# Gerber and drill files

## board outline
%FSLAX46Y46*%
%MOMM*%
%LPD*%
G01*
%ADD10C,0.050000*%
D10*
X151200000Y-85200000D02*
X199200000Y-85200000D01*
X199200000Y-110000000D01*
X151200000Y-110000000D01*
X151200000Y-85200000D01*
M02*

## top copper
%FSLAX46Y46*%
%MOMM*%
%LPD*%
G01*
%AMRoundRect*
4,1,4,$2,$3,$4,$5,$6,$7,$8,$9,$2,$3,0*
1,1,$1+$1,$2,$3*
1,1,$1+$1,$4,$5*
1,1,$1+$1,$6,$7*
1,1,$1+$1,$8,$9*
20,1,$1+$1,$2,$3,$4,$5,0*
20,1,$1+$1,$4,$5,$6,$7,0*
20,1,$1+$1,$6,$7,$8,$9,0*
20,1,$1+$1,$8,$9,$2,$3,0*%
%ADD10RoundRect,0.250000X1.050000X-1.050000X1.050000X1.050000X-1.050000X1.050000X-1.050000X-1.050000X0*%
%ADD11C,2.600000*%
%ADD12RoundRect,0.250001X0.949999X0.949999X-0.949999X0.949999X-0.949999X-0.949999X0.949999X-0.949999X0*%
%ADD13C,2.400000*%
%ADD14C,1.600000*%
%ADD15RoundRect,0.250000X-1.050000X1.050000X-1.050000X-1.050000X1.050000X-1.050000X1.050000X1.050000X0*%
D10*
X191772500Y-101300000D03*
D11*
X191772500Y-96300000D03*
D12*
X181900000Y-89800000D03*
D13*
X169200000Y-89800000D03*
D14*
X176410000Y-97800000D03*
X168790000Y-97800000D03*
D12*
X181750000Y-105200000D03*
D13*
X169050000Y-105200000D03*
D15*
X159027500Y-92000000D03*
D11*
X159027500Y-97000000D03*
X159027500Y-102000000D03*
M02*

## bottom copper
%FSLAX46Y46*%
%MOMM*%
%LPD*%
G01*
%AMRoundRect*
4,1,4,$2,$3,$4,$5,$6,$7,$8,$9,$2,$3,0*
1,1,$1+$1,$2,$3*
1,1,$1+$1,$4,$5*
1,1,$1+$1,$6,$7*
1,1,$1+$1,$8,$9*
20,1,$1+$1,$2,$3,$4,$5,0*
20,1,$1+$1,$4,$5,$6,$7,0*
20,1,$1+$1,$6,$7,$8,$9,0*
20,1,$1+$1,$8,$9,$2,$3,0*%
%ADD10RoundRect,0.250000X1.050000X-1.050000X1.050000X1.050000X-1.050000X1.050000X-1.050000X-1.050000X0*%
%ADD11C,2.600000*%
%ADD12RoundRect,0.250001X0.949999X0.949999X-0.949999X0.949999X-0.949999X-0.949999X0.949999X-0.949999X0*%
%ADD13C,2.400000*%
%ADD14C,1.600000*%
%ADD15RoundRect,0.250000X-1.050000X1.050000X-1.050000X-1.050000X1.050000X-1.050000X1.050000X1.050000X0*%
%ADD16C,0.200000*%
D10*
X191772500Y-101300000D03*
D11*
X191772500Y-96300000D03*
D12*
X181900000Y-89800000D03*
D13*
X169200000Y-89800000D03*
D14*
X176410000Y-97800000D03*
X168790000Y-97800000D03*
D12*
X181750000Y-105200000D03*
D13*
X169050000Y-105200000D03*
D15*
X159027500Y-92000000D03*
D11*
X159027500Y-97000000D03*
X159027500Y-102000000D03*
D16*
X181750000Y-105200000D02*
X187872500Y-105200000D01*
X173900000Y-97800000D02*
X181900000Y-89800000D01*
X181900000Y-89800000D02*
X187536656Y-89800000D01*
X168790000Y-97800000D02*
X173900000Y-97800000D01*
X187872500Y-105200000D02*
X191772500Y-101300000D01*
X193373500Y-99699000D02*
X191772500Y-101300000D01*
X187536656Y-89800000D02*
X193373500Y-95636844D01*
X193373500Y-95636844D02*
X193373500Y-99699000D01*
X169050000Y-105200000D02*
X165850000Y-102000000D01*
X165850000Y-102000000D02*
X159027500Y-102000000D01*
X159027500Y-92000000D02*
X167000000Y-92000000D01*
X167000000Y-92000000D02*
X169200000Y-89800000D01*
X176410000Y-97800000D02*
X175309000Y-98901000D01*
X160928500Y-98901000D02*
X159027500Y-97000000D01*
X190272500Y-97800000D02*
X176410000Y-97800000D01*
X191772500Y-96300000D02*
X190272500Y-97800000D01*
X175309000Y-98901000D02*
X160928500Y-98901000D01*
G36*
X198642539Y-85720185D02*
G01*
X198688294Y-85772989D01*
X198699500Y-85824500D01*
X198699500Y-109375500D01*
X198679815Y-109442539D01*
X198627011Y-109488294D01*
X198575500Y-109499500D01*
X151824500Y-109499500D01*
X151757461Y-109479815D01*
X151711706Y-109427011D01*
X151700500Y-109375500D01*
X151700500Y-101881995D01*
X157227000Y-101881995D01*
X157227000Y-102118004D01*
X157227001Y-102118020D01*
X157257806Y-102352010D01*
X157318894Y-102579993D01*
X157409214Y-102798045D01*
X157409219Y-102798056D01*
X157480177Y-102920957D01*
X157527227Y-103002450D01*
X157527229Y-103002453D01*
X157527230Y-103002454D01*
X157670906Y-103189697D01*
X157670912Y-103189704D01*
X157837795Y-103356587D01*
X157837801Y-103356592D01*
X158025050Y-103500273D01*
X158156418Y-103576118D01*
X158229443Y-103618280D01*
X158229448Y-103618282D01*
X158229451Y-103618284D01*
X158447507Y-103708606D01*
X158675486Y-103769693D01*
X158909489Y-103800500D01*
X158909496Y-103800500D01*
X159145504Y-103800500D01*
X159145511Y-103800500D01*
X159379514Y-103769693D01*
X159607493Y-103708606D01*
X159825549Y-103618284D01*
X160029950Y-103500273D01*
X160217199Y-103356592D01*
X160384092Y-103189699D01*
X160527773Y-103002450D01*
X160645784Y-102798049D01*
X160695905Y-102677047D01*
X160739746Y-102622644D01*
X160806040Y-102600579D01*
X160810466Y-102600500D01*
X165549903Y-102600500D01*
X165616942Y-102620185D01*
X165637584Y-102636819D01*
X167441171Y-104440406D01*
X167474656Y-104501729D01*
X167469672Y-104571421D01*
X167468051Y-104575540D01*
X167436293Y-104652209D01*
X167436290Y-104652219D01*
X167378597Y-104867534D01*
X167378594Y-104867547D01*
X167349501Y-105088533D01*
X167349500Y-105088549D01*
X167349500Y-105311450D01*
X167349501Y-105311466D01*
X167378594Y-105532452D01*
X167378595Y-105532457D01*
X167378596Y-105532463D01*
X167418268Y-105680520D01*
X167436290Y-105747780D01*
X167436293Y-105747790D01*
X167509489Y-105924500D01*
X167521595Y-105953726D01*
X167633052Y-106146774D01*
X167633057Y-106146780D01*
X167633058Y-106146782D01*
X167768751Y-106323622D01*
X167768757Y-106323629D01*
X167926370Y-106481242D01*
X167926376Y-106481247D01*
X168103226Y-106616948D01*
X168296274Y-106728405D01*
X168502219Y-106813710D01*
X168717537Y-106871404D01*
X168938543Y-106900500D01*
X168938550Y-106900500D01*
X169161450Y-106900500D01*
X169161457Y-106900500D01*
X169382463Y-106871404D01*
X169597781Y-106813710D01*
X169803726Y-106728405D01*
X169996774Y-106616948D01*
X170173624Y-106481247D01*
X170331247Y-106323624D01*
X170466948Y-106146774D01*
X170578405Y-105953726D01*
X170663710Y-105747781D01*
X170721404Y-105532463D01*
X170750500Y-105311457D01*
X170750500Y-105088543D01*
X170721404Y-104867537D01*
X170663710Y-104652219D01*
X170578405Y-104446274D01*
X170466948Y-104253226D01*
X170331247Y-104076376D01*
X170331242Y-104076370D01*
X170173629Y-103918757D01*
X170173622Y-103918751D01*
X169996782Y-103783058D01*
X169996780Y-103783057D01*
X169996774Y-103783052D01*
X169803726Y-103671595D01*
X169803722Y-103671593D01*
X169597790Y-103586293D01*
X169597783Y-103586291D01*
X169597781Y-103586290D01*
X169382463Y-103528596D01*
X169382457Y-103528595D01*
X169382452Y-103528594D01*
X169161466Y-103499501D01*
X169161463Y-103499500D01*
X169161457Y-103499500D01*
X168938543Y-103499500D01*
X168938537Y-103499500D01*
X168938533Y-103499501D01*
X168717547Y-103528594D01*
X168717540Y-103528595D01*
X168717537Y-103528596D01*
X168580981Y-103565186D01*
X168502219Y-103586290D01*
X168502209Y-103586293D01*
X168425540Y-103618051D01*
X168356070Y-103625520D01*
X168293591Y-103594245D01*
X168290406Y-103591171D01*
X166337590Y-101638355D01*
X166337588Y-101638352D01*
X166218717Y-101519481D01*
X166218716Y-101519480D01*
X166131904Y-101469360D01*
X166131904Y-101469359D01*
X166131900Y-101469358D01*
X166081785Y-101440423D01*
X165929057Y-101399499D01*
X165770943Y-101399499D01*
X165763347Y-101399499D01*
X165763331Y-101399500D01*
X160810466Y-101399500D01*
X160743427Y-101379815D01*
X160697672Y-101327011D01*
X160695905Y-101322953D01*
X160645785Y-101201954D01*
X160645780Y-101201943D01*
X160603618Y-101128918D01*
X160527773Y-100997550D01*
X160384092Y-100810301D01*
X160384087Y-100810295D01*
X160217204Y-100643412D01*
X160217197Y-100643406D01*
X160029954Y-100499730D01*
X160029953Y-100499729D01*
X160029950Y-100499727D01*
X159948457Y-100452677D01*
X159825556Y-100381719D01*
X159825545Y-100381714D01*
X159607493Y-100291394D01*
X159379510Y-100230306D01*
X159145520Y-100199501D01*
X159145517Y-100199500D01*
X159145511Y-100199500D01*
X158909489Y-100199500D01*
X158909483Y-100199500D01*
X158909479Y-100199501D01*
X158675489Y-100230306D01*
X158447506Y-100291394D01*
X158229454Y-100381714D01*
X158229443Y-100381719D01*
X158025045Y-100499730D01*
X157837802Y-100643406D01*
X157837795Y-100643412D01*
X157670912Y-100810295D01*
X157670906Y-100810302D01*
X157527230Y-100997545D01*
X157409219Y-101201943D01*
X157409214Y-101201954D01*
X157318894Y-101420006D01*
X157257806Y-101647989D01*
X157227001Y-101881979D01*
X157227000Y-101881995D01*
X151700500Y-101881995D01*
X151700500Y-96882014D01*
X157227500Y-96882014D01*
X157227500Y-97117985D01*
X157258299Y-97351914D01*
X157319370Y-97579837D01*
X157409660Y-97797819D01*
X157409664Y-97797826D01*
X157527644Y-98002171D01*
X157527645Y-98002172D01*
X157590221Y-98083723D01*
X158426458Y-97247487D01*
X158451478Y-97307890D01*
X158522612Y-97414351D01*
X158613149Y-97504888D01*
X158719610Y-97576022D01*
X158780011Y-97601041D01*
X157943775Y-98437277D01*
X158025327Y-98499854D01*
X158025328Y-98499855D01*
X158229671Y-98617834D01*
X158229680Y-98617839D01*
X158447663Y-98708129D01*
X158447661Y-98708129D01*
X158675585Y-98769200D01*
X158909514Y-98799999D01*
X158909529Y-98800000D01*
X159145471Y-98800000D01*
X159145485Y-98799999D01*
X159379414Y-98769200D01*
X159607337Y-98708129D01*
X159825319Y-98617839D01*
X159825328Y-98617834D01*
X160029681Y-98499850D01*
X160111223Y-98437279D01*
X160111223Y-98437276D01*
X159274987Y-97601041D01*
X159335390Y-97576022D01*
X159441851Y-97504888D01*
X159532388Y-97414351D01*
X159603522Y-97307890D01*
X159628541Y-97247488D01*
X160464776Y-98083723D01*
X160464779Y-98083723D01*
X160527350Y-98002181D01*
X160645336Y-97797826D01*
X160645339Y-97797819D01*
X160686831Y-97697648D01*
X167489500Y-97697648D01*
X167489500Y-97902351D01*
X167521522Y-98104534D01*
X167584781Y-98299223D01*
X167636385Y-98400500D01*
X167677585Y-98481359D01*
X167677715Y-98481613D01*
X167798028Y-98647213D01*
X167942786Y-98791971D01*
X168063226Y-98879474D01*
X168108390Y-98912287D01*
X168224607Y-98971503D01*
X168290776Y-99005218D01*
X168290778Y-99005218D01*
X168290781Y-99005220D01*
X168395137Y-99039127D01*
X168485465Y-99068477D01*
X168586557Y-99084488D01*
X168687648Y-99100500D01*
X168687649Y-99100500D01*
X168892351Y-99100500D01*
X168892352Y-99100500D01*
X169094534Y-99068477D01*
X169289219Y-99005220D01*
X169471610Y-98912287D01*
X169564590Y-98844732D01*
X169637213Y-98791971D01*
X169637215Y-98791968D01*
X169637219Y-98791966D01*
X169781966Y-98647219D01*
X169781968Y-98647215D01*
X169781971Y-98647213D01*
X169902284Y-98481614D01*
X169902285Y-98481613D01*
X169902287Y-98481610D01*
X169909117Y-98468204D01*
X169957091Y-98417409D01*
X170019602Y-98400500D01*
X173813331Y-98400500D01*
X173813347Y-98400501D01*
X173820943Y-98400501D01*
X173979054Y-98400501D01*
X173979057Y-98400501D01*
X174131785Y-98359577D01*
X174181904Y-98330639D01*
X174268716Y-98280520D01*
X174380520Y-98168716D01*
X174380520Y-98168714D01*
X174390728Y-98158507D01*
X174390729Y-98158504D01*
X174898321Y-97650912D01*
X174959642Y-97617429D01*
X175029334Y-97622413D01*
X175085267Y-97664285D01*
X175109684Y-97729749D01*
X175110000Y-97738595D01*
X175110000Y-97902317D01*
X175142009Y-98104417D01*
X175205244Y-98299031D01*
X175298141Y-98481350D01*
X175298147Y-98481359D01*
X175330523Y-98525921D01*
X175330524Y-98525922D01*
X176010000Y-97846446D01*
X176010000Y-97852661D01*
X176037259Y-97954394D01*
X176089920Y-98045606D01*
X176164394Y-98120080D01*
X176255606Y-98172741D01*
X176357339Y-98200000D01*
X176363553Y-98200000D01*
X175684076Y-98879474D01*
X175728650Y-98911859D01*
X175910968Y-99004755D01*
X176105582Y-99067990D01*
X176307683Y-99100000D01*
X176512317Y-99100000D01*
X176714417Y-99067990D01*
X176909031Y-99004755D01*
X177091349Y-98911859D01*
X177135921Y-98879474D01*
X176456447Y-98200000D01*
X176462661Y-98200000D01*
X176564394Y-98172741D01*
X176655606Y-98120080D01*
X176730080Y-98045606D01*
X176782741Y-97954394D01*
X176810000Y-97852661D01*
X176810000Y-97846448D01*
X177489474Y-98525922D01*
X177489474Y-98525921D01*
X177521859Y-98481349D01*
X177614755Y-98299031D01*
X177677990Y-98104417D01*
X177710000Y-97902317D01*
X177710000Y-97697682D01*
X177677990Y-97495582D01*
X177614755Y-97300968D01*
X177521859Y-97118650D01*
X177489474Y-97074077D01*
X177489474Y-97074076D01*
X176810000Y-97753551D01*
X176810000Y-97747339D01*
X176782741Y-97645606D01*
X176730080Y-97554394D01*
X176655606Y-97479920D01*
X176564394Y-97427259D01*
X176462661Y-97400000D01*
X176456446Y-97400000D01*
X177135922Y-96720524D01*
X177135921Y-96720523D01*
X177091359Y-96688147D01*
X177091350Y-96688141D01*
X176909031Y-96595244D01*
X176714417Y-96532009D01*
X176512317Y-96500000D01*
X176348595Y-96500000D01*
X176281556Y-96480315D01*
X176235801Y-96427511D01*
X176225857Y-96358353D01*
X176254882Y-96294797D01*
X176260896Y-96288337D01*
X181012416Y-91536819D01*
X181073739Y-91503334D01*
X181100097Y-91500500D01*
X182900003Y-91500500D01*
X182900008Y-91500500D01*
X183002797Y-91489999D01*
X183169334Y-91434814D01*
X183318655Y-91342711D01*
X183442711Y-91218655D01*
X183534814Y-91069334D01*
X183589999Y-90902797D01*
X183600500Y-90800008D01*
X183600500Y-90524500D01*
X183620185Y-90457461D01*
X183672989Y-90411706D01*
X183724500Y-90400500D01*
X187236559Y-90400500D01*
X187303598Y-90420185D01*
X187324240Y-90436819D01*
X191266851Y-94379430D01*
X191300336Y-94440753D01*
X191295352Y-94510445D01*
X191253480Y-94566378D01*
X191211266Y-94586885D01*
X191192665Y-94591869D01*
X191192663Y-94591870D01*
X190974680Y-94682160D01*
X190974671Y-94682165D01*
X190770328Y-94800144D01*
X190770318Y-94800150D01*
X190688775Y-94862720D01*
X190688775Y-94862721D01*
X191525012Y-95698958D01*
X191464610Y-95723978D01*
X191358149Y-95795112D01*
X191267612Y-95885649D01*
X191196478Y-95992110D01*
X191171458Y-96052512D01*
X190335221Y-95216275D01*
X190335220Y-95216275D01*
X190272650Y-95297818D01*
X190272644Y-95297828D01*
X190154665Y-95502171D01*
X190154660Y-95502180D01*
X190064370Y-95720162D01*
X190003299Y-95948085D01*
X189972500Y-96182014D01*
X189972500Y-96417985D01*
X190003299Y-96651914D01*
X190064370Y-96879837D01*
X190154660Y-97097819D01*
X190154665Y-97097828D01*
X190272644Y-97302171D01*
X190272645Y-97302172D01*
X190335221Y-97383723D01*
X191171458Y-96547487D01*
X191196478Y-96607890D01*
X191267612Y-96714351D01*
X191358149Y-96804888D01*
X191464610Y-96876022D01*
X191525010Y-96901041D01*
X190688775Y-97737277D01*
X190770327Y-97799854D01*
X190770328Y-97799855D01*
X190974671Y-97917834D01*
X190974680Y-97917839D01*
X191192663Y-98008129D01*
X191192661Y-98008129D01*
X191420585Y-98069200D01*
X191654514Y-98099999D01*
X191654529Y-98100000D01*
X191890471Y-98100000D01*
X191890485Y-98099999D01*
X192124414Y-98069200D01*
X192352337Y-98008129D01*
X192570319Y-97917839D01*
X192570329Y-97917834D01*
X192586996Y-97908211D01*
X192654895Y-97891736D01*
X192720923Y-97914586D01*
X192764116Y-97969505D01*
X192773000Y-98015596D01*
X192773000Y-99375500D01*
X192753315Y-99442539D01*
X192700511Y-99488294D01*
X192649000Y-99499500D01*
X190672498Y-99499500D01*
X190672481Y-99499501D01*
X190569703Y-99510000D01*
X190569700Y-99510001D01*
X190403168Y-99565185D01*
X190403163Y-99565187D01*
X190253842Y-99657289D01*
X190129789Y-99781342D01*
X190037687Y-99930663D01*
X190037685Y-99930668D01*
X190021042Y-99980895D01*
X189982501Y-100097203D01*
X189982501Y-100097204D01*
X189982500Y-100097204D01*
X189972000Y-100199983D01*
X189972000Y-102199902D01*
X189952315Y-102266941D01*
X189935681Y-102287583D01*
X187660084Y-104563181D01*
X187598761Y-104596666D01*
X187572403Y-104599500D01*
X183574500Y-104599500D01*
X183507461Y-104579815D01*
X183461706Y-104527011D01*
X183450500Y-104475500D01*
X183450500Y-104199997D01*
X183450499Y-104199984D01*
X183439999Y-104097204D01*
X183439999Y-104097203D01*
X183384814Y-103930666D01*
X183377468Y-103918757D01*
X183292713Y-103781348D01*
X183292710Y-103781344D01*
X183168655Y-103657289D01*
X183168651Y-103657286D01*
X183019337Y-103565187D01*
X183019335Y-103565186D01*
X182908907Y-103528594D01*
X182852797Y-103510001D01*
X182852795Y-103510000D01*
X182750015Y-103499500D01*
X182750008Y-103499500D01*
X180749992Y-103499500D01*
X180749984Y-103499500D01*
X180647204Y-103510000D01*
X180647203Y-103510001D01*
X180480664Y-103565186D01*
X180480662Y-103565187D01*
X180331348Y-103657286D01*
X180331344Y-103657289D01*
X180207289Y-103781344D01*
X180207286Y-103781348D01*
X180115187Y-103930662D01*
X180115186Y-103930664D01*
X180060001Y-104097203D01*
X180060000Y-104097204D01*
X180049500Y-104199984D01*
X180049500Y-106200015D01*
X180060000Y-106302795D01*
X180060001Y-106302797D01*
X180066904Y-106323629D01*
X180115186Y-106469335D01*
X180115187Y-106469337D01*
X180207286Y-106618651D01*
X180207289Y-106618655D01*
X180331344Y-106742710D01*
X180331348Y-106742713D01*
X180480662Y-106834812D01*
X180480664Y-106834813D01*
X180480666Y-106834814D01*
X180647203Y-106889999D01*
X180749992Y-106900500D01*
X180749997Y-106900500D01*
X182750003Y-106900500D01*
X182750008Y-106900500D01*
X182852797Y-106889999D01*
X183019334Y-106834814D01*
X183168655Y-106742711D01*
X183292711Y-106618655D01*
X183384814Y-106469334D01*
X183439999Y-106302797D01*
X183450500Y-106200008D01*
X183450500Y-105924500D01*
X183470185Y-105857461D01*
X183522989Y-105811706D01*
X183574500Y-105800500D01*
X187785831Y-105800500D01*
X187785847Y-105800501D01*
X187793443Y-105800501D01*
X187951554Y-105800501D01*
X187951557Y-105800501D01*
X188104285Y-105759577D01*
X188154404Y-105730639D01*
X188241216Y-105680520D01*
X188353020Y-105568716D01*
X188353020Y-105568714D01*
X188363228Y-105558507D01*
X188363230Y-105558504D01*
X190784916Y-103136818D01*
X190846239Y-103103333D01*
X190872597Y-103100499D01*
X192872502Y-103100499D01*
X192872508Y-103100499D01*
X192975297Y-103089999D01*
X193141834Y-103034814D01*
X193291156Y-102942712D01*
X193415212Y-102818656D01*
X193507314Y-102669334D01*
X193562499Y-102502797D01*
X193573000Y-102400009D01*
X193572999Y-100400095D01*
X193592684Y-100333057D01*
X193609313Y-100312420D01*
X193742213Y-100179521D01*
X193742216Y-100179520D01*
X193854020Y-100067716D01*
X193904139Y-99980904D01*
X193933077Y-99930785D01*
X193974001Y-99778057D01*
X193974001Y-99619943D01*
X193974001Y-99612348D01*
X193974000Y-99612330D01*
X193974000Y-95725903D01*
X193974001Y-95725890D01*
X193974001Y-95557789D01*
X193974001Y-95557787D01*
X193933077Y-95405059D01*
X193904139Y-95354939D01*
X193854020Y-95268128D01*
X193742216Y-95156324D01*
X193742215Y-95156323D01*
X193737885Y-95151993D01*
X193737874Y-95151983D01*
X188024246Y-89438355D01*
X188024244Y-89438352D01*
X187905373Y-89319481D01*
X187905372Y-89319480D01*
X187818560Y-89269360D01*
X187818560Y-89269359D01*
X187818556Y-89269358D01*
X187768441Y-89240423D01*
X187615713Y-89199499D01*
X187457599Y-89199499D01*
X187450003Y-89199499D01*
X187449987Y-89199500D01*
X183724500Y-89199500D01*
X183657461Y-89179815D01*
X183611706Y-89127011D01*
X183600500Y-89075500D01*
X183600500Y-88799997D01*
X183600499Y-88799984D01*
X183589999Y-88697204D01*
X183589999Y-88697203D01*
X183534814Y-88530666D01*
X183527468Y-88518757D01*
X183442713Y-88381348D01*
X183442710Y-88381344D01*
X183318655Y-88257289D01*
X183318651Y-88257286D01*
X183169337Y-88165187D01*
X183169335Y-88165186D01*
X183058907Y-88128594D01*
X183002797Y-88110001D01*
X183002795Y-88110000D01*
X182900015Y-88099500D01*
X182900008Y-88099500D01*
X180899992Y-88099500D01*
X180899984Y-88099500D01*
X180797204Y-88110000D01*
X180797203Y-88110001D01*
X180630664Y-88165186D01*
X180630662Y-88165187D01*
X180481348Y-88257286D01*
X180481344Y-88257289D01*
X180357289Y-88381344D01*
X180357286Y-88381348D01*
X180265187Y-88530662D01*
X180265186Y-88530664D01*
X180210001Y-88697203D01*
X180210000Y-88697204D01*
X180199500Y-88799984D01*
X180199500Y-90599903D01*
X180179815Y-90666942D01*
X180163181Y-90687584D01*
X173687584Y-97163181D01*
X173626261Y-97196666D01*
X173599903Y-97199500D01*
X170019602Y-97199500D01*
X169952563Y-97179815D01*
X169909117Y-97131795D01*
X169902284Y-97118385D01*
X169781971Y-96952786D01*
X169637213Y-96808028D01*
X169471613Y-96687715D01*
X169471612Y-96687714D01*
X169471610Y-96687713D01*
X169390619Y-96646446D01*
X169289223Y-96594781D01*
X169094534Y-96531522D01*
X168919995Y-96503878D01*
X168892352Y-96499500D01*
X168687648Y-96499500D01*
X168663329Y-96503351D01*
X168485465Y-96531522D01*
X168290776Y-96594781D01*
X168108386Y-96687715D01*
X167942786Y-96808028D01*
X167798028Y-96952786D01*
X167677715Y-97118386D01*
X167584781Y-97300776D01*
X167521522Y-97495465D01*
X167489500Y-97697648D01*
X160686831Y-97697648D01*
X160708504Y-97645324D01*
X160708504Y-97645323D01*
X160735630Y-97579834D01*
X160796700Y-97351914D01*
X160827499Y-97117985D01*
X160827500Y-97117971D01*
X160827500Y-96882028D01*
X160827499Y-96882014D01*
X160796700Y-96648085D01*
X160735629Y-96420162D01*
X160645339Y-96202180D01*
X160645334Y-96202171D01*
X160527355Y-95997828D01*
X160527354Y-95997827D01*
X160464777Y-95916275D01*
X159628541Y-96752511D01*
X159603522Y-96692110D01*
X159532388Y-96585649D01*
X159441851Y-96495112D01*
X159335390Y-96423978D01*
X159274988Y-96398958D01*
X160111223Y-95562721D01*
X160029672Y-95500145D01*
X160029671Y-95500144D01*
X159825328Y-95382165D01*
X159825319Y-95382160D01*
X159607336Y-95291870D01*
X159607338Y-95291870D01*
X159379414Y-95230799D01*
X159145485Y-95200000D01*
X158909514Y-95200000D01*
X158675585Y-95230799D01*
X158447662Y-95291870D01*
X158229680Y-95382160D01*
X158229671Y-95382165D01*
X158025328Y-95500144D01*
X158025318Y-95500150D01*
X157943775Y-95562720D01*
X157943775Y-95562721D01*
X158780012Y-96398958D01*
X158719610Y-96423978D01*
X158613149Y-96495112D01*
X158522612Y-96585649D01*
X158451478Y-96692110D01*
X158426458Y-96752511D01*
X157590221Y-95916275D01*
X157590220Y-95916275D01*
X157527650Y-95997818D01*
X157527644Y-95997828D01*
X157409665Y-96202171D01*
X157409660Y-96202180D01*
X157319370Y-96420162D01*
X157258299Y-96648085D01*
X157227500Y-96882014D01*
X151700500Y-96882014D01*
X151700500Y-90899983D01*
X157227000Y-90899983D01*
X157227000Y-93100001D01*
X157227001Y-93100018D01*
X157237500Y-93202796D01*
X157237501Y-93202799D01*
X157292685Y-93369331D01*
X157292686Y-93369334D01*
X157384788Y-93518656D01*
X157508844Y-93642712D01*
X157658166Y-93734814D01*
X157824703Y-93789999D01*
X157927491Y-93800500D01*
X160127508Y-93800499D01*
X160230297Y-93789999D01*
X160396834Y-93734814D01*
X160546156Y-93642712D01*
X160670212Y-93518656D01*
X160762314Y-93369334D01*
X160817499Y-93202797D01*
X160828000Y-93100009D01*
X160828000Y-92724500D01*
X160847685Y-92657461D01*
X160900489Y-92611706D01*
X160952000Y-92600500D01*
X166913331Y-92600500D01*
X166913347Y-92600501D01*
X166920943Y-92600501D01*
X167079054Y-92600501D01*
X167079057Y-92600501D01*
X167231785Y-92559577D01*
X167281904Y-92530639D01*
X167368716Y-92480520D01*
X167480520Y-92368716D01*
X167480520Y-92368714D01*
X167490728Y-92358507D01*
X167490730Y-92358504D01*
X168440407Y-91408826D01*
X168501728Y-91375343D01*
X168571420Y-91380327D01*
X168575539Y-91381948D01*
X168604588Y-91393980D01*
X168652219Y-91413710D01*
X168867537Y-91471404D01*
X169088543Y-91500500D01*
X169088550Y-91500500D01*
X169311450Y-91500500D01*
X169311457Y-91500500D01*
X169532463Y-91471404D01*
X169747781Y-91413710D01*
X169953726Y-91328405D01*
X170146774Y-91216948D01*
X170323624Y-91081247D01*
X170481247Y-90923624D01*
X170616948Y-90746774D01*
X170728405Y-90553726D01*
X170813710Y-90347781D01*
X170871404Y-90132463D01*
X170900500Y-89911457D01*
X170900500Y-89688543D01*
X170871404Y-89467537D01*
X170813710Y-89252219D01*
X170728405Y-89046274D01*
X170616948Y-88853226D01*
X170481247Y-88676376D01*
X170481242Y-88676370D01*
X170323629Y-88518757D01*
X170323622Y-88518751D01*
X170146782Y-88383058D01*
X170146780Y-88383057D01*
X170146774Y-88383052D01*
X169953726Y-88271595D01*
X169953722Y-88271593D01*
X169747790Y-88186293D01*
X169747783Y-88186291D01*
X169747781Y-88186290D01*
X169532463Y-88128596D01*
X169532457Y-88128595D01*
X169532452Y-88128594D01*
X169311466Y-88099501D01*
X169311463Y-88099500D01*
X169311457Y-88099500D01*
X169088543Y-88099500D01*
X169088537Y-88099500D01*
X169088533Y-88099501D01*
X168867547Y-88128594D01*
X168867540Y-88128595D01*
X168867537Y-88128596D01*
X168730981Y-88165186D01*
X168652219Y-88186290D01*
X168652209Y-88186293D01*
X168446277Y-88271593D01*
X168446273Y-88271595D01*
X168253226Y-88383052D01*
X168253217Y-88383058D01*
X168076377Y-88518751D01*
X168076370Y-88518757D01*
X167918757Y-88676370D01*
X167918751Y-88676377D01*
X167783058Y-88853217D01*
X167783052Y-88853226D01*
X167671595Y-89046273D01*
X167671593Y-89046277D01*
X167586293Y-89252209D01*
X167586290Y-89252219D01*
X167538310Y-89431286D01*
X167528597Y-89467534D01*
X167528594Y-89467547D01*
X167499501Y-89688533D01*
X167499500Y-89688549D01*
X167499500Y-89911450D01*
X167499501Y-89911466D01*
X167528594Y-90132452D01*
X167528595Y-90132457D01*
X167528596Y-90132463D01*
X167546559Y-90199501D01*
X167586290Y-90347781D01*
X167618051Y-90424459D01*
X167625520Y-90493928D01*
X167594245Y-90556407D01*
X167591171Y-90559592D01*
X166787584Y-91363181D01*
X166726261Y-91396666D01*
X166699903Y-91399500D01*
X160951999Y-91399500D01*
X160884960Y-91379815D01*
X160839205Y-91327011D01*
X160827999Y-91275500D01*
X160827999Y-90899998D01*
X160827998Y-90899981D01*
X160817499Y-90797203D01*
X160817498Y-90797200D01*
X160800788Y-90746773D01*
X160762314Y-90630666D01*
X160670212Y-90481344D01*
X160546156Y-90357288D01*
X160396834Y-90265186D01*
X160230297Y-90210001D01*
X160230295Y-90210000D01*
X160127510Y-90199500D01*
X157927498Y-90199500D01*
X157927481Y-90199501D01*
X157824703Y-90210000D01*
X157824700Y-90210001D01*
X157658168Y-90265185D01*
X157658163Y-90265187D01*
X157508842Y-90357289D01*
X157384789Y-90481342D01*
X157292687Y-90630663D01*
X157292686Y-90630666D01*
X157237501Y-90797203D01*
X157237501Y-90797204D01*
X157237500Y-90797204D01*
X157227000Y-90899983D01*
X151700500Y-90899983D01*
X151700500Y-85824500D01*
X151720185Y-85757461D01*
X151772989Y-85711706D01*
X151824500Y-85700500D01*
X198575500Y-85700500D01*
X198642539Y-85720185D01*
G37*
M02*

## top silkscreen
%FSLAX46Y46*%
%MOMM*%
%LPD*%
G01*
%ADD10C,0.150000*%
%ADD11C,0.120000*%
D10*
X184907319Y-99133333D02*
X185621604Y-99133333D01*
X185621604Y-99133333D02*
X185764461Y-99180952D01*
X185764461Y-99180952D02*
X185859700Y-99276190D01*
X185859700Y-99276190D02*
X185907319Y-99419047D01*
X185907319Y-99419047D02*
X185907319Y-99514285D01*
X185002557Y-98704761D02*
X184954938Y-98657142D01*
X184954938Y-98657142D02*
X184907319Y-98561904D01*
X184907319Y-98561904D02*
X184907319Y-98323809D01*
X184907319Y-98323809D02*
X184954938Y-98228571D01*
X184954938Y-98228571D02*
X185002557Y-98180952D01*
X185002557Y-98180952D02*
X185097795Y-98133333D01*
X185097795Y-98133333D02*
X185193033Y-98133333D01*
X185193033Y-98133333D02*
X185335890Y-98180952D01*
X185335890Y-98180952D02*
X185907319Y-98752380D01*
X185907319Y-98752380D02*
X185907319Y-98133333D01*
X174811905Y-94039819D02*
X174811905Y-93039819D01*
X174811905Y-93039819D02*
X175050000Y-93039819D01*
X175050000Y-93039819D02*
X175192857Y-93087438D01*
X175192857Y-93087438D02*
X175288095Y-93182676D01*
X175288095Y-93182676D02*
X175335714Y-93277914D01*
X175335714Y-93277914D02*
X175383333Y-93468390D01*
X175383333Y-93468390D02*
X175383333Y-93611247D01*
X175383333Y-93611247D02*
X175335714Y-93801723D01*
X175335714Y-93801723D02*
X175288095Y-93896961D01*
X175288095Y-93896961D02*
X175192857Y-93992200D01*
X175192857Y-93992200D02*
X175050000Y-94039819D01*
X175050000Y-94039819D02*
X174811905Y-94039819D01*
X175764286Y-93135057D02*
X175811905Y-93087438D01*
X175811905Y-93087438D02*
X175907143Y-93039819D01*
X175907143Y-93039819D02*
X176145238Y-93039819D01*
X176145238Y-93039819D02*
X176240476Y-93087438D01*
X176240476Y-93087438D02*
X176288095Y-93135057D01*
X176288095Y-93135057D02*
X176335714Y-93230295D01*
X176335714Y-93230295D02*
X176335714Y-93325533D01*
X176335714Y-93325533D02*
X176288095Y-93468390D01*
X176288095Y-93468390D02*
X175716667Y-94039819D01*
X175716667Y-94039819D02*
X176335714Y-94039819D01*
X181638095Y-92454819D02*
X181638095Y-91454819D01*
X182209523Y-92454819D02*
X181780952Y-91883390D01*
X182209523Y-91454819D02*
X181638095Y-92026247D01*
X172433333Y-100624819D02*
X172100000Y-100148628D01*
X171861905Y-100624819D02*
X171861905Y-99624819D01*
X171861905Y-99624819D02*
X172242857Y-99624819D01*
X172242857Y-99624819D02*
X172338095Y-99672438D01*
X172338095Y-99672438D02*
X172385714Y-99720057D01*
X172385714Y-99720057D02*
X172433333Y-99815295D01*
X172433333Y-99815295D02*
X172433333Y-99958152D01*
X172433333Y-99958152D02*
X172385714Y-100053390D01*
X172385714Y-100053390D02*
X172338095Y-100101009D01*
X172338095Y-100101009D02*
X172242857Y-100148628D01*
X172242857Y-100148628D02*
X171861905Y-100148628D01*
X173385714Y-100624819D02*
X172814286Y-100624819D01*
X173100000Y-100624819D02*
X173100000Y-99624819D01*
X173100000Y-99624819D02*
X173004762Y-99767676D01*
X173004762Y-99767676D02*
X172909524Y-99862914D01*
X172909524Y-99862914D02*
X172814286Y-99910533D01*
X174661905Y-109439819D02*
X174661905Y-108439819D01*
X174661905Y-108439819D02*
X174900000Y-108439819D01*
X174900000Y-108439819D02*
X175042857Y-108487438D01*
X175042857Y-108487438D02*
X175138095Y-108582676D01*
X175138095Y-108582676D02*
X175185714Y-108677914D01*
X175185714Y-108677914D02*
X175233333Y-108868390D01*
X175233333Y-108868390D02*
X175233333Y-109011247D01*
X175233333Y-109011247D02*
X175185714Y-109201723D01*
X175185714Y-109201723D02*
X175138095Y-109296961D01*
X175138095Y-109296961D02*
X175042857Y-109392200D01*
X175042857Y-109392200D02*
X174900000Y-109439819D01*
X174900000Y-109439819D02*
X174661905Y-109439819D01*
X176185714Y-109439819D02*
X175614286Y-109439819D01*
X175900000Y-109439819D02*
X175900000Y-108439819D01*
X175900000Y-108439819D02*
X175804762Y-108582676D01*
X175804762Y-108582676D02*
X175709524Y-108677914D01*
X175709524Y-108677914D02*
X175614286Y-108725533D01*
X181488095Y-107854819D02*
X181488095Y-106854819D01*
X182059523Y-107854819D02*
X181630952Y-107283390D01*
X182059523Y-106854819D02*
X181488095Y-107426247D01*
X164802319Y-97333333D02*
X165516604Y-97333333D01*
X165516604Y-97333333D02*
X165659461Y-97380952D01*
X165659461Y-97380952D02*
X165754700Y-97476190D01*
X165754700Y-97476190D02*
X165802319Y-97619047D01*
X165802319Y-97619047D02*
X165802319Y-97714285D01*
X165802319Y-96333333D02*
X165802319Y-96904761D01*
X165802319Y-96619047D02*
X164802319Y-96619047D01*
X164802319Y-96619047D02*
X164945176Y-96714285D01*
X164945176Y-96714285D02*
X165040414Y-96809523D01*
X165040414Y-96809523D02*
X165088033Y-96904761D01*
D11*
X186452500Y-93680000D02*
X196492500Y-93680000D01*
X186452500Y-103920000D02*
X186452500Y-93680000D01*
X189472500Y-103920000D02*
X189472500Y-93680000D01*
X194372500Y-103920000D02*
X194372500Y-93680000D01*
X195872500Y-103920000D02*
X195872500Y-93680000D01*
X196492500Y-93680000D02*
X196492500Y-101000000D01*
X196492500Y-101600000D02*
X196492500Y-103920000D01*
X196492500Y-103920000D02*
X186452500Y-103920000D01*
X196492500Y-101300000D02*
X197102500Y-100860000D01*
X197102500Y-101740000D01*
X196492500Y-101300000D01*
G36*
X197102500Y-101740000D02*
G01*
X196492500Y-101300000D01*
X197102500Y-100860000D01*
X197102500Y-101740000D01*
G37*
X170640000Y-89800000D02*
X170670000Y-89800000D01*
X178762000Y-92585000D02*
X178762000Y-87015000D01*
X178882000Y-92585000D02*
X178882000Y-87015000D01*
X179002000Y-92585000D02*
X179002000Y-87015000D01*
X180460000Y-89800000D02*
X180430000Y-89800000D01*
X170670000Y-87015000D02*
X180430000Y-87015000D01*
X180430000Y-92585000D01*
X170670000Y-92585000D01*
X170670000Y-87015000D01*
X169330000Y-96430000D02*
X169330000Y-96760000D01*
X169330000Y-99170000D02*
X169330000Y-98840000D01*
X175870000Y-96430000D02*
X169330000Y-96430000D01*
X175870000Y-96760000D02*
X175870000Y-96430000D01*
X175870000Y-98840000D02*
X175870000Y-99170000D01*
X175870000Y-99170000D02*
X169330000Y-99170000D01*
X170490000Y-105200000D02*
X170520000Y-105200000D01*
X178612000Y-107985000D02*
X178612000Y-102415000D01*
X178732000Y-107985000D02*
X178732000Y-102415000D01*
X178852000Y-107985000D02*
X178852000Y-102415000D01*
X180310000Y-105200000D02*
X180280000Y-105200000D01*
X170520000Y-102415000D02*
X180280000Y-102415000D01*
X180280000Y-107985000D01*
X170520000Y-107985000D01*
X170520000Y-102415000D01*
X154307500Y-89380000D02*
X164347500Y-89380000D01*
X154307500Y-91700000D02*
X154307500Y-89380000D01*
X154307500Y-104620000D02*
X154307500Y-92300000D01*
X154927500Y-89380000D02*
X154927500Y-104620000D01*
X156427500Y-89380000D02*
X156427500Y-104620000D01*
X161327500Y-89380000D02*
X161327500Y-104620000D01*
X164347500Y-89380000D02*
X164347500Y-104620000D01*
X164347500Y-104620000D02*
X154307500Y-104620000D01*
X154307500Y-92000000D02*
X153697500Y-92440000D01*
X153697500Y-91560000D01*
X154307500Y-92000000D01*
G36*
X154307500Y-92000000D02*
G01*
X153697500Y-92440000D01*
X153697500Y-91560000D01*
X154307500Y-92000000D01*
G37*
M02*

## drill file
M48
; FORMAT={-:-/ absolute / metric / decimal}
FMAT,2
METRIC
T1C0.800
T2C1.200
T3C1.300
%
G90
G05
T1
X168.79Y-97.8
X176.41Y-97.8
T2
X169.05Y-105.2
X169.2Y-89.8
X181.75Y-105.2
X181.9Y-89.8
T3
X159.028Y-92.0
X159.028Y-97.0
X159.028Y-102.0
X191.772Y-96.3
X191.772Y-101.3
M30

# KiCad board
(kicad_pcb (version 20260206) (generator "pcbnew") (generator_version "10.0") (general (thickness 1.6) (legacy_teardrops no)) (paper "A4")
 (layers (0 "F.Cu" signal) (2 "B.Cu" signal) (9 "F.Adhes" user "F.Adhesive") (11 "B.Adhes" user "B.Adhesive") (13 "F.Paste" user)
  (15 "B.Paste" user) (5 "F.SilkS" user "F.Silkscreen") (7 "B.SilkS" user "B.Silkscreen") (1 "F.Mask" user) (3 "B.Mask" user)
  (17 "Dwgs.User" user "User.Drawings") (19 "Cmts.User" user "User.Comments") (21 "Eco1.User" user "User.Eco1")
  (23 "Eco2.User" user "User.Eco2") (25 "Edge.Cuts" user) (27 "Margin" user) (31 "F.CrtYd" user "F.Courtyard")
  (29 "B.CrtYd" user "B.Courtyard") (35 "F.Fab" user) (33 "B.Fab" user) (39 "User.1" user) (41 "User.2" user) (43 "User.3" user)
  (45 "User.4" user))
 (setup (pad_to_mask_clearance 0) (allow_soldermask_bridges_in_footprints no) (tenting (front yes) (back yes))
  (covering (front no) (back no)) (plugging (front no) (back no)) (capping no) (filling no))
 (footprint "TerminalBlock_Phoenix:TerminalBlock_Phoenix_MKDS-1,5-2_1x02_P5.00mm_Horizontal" (layer "F.Cu") (at 191.7725 101.3 90)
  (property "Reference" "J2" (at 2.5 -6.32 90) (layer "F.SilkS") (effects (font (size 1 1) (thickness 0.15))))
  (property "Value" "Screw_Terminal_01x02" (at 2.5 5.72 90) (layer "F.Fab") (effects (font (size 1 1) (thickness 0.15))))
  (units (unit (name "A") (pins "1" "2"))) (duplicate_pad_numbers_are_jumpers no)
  (fp_line (start 7.62 -5.32) (end 7.62 4.72) (stroke (width 0.12) (type solid)) (layer "F.SilkS"))
  (fp_line (start -2.62 -5.32) (end 7.62 -5.32) (stroke (width 0.12) (type solid)) (layer "F.SilkS"))
  (fp_line (start -2.62 -2.3) (end 7.62 -2.3) (stroke (width 0.12) (type solid)) (layer "F.SilkS"))
  (fp_line (start -2.62 2.6) (end 7.62 2.6) (stroke (width 0.12) (type solid)) (layer "F.SilkS"))
  (fp_line (start -2.62 4.1) (end 7.62 4.1) (stroke (width 0.12) (type solid)) (layer "F.SilkS"))
  (fp_line (start 7.62 4.72) (end 0.3 4.72) (stroke (width 0.12) (type solid)) (layer "F.SilkS"))
  (fp_line (start -0.3 4.72) (end -2.62 4.72) (stroke (width 0.12) (type solid)) (layer "F.SilkS"))
  (fp_line (start -2.62 4.72) (end -2.62 -5.32) (stroke (width 0.12) (type solid)) (layer "F.SilkS"))
  (fp_poly (pts (xy 0 4.72) (xy 0.44 5.33) (xy -0.44 5.33)) (stroke (width 0.12) (type solid)) (fill yes) (layer "F.SilkS"))
  (pad "1" thru_hole roundrect (at 0 0 90) (size 2.6 2.6) (drill 1.3) (layers "*.Cu" "*.Mask") (remove_unused_layers no)
   (roundrect_rratio 0.096154) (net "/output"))
  (pad "2" thru_hole circle (at 5 0 90) (size 2.6 2.6) (drill 1.3) (layers "*.Cu" "*.Mask") (remove_unused_layers no) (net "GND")))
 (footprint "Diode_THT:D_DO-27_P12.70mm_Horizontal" (layer "F.Cu") (at 181.9 89.8 180)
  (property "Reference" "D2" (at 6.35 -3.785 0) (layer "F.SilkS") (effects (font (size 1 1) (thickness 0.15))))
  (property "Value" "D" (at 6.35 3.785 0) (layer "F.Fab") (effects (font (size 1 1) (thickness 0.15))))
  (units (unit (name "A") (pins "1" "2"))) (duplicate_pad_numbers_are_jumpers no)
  (fp_line (start 11.26 0) (end 11.23 0) (stroke (width 0.12) (type solid)) (layer "F.SilkS"))
  (fp_line (start 3.138 -2.785) (end 3.138 2.785) (stroke (width 0.12) (type solid)) (layer "F.SilkS"))
  (fp_line (start 3.018 -2.785) (end 3.018 2.785) (stroke (width 0.12) (type solid)) (layer "F.SilkS"))
  (fp_line (start 2.898 -2.785) (end 2.898 2.785) (stroke (width 0.12) (type solid)) (layer "F.SilkS"))
  (fp_line (start 1.44 0) (end 1.47 0) (stroke (width 0.12) (type solid)) (layer "F.SilkS"))
  (fp_rect (start 1.47 -2.785) (end 11.23 2.785) (stroke (width 0.12) (type solid)) (fill no) (layer "F.SilkS"))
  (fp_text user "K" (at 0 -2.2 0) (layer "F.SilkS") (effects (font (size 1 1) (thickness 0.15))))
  (pad "1" thru_hole roundrect (at 0 0 180) (size 2.4 2.4) (drill 1.2) (layers "*.Cu" "*.Mask") (remove_unused_layers no)
   (roundrect_rratio 0.104167) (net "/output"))
  (pad "2" thru_hole circle (at 12.7 0 180) (size 2.4 2.4) (drill 1.2) (layers "*.Cu" "*.Mask") (remove_unused_layers no) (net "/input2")))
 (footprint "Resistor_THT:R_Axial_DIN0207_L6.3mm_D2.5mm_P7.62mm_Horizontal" (layer "F.Cu") (at 176.41 97.8 180)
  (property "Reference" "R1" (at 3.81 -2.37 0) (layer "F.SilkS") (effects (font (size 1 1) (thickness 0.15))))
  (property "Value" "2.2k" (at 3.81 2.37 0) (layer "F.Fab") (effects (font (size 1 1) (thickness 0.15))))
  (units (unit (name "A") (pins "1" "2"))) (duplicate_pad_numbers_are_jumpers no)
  (fp_line (start 7.08 1.37) (end 7.08 1.04) (stroke (width 0.12) (type solid)) (layer "F.SilkS"))
  (fp_line (start 7.08 -1.37) (end 7.08 -1.04) (stroke (width 0.12) (type solid)) (layer "F.SilkS"))
  (fp_line (start 0.54 1.37) (end 7.08 1.37) (stroke (width 0.12) (type solid)) (layer "F.SilkS"))
  (fp_line (start 0.54 1.04) (end 0.54 1.37) (stroke (width 0.12) (type solid)) (layer "F.SilkS"))
  (fp_line (start 0.54 -1.04) (end 0.54 -1.37) (stroke (width 0.12) (type solid)) (layer "F.SilkS"))
  (fp_line (start 0.54 -1.37) (end 7.08 -1.37) (stroke (width 0.12) (type solid)) (layer "F.SilkS"))
  (pad "1" thru_hole circle (at 0 0 180) (size 1.6 1.6) (drill 0.8) (layers "*.Cu" "*.Mask") (remove_unused_layers no) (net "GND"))
  (pad "2" thru_hole circle (at 7.62 0 180) (size 1.6 1.6) (drill 0.8) (layers "*.Cu" "*.Mask") (remove_unused_layers no) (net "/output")))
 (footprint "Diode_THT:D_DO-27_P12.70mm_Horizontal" (layer "F.Cu") (at 181.75 105.2 180)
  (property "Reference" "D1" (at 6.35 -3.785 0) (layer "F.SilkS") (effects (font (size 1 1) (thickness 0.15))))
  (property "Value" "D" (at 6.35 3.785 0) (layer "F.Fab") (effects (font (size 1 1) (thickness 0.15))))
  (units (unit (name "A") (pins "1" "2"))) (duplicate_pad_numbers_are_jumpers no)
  (fp_line (start 11.26 0) (end 11.23 0) (stroke (width 0.12) (type solid)) (layer "F.SilkS"))
  (fp_line (start 3.138 -2.785) (end 3.138 2.785) (stroke (width 0.12) (type solid)) (layer "F.SilkS"))
  (fp_line (start 3.018 -2.785) (end 3.018 2.785) (stroke (width 0.12) (type solid)) (layer "F.SilkS"))
  (fp_line (start 2.898 -2.785) (end 2.898 2.785) (stroke (width 0.12) (type solid)) (layer "F.SilkS"))
  (fp_line (start 1.44 0) (end 1.47 0) (stroke (width 0.12) (type solid)) (layer "F.SilkS"))
  (fp_rect (start 1.47 -2.785) (end 11.23 2.785) (stroke (width 0.12) (type solid)) (fill no) (layer "F.SilkS"))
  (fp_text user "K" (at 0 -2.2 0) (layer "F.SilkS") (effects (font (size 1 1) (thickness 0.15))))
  (pad "1" thru_hole roundrect (at 0 0 180) (size 2.4 2.4) (drill 1.2) (layers "*.Cu" "*.Mask") (remove_unused_layers no)
   (roundrect_rratio 0.104167) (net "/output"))
  (pad "2" thru_hole circle (at 12.7 0 180) (size 2.4 2.4) (drill 1.2) (layers "*.Cu" "*.Mask") (remove_unused_layers no) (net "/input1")))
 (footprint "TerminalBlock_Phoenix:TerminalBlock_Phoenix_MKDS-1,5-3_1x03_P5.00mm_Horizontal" (layer "F.Cu") (at 159.0275 92 -90)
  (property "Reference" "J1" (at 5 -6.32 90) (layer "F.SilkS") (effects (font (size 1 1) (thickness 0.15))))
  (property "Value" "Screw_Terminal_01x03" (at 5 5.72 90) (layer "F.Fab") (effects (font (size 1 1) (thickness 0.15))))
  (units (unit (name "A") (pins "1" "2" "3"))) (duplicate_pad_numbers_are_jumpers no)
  (fp_line (start -2.62 4.72) (end -2.62 -5.32) (stroke (width 0.12) (type solid)) (layer "F.SilkS"))
  (fp_line (start -0.3 4.72) (end -2.62 4.72) (stroke (width 0.12) (type solid)) (layer "F.SilkS"))
  (fp_line (start 12.62 4.72) (end 0.3 4.72) (stroke (width 0.12) (type solid)) (layer "F.SilkS"))
  (fp_line (start -2.62 4.1) (end 12.62 4.1) (stroke (width 0.12) (type solid)) (layer "F.SilkS"))
  (fp_line (start -2.62 2.6) (end 12.62 2.6) (stroke (width 0.12) (type solid)) (layer "F.SilkS"))
  (fp_line (start -2.62 -2.3) (end 12.62 -2.3) (stroke (width 0.12) (type solid)) (layer "F.SilkS"))
  (fp_line (start -2.62 -5.32) (end 12.62 -5.32) (stroke (width 0.12) (type solid)) (layer "F.SilkS"))
  (fp_line (start 12.62 -5.32) (end 12.62 4.72) (stroke (width 0.12) (type solid)) (layer "F.SilkS"))
  (fp_poly (pts (xy 0 4.72) (xy 0.44 5.33) (xy -0.44 5.33)) (stroke (width 0.12) (type solid)) (fill yes) (layer "F.SilkS"))
  (pad "1" thru_hole roundrect (at 0 0 270) (size 2.6 2.6) (drill 1.3) (layers "*.Cu" "*.Mask") (remove_unused_layers no)
   (roundrect_rratio 0.096154) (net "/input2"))
  (pad "2" thru_hole circle (at 5 0 270) (size 2.6 2.6) (drill 1.3) (layers "*.Cu" "*.Mask") (remove_unused_layers no) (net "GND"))
  (pad "3" thru_hole circle (at 10 0 270) (size 2.6 2.6) (drill 1.3) (layers "*.Cu" "*.Mask") (remove_unused_layers no) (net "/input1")))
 (gr_rect (start 151.2 85.2) (end 199.2 110) (stroke (width 0.05) (type default)) (fill no) (layer "Edge.Cuts"))
 (segment (start 181.75 105.2) (end 187.8725 105.2) (width 0.2) (layer "B.Cu") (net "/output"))
 (segment (start 173.9 97.8) (end 181.9 89.8) (width 0.2) (layer "B.Cu") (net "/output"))
 (segment (start 181.9 89.8) (end 187.536656 89.8) (width 0.2) (layer "B.Cu") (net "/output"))
 (segment (start 168.79 97.8) (end 173.9 97.8) (width 0.2) (layer "B.Cu") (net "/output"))
 (segment (start 187.8725 105.2) (end 191.7725 101.3) (width 0.2) (layer "B.Cu") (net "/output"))
 (segment (start 193.3735 99.699) (end 191.7725 101.3) (width 0.2) (layer "B.Cu") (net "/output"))
 (segment (start 187.536656 89.8) (end 193.3735 95.636844) (width 0.2) (layer "B.Cu") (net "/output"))
 (segment (start 193.3735 95.636844) (end 193.3735 99.699) (width 0.2) (layer "B.Cu") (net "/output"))
 (segment (start 169.05 105.2) (end 165.85 102) (width 0.2) (layer "B.Cu") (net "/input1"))
 (segment (start 165.85 102) (end 159.0275 102) (width 0.2) (layer "B.Cu") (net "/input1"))
 (segment (start 159.0275 92) (end 167 92) (width 0.2) (layer "B.Cu") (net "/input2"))
 (segment (start 167 92) (end 169.2 89.8) (width 0.2) (layer "B.Cu") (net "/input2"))
 (segment (start 176.41 97.8) (end 175.309 98.901) (width 0.2) (layer "B.Cu") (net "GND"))
 (segment (start 160.9285 98.901) (end 159.0275 97) (width 0.2) (layer "B.Cu") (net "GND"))
 (segment (start 190.2725 97.8) (end 176.41 97.8) (width 0.2) (layer "B.Cu") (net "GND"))
 (segment (start 191.7725 96.3) (end 190.2725 97.8) (width 0.2) (layer "B.Cu") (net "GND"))
 (segment (start 175.309 98.901) (end 160.9285 98.901) (width 0.2) (layer "B.Cu") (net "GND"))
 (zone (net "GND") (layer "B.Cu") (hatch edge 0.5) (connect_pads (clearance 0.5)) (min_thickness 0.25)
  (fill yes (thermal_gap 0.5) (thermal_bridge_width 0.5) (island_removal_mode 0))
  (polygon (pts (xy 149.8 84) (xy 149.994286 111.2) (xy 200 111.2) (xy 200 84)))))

